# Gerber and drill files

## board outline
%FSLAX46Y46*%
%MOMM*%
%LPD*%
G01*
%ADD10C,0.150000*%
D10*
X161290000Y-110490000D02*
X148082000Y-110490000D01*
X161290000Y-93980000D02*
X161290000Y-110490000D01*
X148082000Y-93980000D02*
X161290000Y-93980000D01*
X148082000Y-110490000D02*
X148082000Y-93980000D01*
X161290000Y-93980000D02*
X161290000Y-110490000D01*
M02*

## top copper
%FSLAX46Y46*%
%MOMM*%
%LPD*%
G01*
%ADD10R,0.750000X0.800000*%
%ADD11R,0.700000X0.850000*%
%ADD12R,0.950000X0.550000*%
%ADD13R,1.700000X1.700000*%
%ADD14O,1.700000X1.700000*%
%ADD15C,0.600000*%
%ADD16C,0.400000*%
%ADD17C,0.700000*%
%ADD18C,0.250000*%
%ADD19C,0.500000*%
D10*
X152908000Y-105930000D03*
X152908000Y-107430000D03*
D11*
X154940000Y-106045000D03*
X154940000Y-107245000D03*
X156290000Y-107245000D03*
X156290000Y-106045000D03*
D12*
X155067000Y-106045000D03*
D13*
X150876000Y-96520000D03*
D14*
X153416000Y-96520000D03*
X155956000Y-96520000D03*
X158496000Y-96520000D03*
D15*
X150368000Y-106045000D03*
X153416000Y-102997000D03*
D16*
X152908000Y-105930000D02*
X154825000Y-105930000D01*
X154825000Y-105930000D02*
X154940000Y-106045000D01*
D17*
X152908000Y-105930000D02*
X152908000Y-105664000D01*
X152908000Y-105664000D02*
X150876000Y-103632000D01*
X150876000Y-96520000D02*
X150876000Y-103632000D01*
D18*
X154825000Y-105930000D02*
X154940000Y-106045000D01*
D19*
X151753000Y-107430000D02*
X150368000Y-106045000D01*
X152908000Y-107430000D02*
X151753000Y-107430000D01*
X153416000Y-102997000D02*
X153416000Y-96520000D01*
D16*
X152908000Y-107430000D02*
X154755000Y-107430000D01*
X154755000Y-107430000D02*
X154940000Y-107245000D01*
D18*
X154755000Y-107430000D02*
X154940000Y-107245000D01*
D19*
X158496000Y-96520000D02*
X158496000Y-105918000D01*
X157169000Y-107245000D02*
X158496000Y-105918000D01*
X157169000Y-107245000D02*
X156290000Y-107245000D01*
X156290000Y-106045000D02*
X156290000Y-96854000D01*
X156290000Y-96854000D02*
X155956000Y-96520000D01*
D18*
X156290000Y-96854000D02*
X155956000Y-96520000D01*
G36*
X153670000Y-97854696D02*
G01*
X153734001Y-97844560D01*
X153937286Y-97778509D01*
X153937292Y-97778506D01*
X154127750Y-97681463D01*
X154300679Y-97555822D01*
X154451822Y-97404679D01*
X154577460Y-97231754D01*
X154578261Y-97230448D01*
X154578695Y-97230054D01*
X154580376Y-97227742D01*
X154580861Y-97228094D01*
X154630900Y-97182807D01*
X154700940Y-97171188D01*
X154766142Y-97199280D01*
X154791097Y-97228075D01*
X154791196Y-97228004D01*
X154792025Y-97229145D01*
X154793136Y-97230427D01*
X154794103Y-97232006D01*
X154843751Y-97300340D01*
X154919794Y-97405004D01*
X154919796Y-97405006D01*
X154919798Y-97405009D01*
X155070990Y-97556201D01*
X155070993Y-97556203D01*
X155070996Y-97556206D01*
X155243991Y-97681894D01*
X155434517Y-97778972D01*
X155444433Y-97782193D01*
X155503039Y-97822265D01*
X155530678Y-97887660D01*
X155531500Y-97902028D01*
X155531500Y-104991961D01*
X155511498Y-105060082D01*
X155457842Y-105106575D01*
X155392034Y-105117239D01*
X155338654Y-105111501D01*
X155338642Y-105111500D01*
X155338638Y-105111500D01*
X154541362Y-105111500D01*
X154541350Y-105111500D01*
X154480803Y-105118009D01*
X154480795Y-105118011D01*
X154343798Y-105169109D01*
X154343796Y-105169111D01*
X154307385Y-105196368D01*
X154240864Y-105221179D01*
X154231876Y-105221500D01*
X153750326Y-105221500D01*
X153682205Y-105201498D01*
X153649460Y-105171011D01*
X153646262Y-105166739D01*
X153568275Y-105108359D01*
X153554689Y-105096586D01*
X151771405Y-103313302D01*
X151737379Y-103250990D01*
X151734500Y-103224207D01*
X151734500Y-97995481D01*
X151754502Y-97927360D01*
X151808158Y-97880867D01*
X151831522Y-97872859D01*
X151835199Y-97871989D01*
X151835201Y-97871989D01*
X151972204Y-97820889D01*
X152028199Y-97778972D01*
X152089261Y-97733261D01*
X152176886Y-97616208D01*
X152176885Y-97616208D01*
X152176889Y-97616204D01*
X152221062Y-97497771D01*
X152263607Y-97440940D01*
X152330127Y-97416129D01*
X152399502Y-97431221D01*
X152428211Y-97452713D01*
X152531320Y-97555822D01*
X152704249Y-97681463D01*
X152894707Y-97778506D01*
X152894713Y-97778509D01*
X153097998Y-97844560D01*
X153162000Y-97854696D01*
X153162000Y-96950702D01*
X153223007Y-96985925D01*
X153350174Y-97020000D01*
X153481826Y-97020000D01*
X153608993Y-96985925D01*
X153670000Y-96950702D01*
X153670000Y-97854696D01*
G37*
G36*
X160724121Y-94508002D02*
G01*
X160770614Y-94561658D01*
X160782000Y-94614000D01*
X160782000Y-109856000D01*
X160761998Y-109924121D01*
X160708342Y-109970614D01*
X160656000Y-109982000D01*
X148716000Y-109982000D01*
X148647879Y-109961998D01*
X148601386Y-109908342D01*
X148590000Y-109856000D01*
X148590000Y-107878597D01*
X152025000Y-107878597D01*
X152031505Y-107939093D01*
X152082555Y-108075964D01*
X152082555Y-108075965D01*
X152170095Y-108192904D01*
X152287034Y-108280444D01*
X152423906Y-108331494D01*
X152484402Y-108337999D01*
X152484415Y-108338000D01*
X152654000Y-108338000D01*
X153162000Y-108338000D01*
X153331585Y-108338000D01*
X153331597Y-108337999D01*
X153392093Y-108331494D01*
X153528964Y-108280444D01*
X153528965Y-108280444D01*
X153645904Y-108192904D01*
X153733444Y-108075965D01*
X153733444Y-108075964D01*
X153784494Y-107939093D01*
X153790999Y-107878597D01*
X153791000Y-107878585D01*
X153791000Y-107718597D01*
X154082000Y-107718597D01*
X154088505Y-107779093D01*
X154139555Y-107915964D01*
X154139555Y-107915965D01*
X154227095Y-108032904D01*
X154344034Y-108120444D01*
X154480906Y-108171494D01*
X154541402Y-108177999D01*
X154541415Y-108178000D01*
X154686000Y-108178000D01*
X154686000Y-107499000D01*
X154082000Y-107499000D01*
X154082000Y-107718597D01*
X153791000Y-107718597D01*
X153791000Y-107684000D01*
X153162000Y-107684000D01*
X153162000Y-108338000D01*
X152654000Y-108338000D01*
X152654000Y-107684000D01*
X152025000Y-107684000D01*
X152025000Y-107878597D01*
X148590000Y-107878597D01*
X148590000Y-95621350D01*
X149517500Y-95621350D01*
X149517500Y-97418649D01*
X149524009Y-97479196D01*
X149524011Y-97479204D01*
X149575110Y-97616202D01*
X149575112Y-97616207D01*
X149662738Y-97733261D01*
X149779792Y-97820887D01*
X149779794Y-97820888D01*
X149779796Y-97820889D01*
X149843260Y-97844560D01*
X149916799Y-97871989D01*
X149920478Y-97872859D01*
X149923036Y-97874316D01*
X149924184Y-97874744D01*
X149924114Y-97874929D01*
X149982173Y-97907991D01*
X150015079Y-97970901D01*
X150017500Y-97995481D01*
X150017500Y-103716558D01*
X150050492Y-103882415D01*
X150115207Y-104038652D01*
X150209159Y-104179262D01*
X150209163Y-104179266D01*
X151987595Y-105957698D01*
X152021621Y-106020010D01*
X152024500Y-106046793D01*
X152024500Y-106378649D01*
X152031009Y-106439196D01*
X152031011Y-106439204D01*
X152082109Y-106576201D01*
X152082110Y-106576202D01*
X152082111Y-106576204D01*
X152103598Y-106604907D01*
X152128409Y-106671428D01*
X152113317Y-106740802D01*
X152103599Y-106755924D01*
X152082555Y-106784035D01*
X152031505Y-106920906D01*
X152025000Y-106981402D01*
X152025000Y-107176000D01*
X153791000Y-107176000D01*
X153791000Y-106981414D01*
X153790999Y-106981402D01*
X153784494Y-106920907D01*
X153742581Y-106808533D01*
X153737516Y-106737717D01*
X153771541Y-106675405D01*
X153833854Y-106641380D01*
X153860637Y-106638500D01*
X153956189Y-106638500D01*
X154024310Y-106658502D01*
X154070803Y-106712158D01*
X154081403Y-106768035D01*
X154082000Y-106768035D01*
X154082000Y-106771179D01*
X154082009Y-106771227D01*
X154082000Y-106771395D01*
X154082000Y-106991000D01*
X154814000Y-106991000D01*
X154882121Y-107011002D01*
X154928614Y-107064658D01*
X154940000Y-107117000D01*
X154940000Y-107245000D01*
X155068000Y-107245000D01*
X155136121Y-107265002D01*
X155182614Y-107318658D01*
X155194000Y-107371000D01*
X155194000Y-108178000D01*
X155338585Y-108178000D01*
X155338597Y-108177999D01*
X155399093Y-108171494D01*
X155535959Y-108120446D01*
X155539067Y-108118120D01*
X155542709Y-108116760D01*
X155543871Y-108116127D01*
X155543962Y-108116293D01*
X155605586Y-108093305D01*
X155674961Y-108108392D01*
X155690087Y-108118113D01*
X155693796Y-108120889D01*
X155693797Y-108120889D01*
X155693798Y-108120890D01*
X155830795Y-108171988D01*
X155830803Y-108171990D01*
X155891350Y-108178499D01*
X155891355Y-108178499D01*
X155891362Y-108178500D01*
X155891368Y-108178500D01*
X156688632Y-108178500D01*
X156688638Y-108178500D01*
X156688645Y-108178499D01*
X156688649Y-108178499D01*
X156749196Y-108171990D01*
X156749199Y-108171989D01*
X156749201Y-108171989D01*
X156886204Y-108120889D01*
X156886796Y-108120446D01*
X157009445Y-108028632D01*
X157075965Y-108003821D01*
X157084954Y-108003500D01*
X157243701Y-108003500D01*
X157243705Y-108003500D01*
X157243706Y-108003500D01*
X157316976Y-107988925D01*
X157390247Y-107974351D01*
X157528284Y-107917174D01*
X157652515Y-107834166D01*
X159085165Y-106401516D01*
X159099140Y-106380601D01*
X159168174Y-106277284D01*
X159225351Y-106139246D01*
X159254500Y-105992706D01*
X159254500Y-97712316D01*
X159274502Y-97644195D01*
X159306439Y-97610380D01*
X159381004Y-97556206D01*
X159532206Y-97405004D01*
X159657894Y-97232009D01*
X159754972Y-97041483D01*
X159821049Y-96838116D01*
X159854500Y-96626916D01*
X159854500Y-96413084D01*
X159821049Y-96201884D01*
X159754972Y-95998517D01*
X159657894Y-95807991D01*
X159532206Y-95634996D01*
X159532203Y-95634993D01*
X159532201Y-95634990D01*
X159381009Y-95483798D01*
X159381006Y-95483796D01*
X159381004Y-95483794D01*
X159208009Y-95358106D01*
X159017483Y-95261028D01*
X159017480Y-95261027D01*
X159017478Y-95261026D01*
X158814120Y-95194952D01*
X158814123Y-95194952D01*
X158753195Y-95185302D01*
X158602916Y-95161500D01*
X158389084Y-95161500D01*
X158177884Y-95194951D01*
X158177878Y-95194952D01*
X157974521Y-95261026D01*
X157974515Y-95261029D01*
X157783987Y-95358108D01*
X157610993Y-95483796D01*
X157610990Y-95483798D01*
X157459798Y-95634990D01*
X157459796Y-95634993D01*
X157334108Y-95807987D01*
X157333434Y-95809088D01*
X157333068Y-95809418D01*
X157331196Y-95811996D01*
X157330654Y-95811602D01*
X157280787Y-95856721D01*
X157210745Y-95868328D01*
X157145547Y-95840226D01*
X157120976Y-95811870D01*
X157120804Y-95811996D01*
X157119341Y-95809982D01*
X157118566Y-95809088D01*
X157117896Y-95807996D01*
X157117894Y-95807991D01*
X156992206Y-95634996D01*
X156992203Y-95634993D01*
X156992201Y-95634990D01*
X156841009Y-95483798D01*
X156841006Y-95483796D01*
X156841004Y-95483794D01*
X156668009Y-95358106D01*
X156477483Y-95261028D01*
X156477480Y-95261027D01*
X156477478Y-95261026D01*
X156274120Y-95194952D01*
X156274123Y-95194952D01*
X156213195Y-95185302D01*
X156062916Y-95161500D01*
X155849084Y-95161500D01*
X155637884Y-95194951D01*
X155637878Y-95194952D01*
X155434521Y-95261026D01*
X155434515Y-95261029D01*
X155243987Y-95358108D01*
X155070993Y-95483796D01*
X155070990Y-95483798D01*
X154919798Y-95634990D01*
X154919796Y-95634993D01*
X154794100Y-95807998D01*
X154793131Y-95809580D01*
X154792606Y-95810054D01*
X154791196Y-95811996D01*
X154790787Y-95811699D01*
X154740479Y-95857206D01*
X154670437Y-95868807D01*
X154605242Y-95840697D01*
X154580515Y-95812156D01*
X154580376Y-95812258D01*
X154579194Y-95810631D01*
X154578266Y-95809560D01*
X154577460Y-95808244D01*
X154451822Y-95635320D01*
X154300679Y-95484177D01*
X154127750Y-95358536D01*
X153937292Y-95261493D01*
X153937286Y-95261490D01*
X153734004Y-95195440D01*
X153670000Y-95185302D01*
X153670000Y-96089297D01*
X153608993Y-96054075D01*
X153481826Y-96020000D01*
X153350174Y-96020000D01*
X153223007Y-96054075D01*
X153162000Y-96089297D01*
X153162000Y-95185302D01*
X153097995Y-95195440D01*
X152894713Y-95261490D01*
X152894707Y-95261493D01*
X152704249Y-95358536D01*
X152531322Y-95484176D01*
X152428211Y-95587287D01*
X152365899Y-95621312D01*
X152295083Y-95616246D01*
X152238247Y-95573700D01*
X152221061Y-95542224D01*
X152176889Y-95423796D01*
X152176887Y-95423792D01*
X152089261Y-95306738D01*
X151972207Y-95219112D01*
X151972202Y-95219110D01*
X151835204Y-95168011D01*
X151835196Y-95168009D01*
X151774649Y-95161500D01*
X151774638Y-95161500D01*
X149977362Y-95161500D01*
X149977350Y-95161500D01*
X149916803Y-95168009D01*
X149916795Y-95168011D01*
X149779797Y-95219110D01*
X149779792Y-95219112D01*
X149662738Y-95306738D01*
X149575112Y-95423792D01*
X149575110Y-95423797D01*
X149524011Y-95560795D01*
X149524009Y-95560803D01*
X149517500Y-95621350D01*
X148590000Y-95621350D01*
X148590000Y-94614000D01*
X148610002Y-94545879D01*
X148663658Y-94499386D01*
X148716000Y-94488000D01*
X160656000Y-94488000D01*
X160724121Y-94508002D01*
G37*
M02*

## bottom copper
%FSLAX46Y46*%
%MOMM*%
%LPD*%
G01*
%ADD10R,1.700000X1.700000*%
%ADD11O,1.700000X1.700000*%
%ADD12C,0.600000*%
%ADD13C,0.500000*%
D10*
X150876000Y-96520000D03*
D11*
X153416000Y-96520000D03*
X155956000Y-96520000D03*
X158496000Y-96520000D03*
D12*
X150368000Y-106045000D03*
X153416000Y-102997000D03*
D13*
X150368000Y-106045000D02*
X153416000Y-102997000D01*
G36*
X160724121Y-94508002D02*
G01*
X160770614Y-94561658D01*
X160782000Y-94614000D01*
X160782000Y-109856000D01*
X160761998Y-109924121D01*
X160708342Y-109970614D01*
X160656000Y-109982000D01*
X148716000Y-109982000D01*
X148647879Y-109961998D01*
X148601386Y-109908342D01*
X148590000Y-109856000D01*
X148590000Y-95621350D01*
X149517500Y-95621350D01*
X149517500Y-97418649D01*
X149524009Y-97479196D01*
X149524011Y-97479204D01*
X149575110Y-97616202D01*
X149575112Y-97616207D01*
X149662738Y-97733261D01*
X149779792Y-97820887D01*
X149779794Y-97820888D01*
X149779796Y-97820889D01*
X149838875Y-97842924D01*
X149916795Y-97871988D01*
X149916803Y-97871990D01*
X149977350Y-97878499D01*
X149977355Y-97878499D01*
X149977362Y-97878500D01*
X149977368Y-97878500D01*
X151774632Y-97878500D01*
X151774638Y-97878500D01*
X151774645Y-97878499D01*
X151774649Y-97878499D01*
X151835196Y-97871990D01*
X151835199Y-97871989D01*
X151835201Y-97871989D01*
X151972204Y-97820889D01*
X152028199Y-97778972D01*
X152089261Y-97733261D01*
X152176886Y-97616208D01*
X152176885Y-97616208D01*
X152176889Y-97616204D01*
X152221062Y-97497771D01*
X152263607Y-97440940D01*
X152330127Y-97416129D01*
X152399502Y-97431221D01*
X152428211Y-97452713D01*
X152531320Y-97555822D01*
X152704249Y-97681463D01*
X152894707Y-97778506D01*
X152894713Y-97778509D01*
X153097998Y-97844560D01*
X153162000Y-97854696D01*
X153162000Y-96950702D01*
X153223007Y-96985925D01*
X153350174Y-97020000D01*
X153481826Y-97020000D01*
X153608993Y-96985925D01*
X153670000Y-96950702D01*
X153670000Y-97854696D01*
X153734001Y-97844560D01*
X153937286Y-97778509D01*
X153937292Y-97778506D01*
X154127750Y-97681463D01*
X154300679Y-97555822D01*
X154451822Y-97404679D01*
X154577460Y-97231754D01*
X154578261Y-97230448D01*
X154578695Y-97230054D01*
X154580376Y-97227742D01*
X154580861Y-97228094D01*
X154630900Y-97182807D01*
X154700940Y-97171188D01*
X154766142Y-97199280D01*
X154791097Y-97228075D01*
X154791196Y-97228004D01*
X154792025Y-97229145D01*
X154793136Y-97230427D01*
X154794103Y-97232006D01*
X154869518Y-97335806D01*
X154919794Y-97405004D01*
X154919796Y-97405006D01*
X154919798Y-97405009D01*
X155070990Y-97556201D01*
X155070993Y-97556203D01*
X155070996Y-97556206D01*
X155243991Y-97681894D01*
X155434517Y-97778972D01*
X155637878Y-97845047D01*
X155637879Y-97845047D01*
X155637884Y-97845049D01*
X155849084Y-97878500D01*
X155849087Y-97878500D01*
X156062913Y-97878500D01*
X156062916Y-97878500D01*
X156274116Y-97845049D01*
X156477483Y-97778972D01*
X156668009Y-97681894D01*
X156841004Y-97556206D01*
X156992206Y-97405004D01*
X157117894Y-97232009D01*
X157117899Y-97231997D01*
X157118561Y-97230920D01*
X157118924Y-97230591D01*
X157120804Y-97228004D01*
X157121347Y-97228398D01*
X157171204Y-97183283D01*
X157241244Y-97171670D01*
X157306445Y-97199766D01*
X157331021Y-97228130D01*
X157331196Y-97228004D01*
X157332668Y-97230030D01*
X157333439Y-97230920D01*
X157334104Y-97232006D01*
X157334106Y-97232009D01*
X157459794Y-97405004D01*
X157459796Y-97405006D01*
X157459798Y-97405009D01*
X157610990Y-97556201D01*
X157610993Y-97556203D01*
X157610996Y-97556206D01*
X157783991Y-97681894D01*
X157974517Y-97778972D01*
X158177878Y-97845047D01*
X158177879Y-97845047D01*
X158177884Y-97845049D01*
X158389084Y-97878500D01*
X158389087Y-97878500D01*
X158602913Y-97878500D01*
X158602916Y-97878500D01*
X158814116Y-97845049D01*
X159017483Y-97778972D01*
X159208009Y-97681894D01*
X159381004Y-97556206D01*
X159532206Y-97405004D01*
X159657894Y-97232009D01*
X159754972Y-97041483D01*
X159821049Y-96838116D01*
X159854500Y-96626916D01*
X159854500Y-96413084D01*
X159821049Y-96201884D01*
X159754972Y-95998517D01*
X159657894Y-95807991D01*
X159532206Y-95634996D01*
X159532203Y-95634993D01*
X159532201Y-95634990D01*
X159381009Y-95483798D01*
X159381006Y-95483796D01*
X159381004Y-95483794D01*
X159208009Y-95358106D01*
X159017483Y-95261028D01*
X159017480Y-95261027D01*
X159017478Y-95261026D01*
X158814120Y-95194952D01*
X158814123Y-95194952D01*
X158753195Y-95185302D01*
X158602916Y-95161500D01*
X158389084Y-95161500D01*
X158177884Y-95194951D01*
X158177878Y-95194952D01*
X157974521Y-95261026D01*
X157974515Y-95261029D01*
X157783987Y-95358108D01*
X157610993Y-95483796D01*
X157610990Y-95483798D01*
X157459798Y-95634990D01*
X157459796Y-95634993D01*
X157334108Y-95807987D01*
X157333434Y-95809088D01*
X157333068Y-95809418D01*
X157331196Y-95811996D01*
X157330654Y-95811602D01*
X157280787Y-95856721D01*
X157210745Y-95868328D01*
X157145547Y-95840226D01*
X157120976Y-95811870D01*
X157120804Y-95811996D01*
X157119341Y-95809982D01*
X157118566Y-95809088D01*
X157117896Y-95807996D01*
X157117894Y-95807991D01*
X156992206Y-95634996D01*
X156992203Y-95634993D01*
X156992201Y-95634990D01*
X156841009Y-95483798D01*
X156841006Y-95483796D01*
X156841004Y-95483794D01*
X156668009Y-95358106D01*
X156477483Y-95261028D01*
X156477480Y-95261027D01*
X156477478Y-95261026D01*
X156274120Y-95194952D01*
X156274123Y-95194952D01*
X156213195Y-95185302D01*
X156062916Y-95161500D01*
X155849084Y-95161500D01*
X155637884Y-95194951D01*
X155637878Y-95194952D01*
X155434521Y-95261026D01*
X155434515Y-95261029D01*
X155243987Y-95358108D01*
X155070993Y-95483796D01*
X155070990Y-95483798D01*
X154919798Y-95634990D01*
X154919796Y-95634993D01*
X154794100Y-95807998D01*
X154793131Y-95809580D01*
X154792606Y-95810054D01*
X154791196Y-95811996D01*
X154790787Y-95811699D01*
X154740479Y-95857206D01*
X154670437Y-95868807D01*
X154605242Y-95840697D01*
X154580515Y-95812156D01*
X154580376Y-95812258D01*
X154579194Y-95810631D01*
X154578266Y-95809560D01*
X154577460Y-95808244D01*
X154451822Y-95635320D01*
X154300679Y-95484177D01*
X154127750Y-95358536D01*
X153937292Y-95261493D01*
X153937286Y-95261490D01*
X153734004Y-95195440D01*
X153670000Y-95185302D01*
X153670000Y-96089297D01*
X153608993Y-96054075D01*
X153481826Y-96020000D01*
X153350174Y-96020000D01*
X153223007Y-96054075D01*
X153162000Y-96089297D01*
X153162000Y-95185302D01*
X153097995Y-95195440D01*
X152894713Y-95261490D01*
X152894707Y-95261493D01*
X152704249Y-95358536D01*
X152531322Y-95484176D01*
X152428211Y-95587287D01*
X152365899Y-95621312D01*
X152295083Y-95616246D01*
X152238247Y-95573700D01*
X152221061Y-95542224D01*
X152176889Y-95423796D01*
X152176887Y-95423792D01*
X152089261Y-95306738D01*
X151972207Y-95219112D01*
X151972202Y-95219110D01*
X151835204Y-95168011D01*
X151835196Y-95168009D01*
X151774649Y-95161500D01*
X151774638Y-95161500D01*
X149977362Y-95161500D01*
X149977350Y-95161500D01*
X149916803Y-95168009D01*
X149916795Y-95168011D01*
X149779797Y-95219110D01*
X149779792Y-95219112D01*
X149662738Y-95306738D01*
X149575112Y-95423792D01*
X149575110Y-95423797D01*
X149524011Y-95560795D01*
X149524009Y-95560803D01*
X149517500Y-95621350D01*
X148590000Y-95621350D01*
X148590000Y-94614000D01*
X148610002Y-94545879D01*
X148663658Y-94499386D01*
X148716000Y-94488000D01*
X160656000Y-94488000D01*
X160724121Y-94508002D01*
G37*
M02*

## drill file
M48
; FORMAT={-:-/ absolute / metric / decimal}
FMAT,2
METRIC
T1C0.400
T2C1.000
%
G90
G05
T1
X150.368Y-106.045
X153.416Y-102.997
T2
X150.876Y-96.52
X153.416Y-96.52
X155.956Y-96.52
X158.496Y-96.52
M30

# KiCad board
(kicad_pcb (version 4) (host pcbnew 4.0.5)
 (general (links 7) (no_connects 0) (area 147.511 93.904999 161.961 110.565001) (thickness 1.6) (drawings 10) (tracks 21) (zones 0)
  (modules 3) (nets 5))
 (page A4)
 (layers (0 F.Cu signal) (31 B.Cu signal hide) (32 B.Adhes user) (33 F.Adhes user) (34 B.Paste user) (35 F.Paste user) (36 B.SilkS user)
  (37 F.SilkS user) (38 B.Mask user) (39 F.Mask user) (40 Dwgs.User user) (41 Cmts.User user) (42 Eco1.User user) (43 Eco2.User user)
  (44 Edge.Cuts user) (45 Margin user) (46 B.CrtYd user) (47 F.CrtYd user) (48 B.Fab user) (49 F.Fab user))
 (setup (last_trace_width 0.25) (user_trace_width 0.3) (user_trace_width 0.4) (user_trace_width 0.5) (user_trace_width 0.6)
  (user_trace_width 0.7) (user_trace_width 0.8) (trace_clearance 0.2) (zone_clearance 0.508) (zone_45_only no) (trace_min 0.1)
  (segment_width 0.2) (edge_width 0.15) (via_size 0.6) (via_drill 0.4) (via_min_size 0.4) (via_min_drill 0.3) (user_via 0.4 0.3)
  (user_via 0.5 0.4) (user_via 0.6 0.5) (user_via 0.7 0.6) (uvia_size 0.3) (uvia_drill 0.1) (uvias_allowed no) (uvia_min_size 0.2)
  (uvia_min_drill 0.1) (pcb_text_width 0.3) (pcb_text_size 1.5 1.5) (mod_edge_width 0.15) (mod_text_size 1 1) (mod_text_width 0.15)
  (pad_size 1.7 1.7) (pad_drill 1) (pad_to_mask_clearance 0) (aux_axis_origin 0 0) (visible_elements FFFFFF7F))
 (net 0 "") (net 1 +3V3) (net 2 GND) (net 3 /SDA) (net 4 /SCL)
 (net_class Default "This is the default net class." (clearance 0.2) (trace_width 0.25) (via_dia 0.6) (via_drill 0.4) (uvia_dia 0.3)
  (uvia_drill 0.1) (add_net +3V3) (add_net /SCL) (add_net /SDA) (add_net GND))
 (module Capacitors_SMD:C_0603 (layer F.Cu) (at 152.908 106.68 270)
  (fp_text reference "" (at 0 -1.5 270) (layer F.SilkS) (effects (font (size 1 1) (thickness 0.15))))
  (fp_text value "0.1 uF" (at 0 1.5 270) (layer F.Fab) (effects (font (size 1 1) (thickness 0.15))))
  (pad 1 smd rect (at -0.75 0 270) (size 0.8 0.75) (layers F.Cu F.Paste F.Mask) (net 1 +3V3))
  (pad 2 smd rect (at 0.75 0 270) (size 0.8 0.75) (layers F.Cu F.Paste F.Mask) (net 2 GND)))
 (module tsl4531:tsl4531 (layer F.Cu) (at 154.94 106.045)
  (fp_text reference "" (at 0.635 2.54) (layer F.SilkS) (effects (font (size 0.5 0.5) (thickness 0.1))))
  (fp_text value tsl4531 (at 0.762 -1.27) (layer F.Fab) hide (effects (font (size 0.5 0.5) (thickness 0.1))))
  (pad 1 smd rect (at 0 0) (size 0.7 0.85) (layers F.Cu F.Paste F.Mask) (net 1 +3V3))
  (pad 2 smd rect (at 0 1.2) (size 0.7 0.85) (layers F.Cu F.Paste F.Mask) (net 2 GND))
  (pad 3 smd rect (at 1.35 1.2) (size 0.7 0.85) (layers F.Cu F.Paste F.Mask) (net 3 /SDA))
  (pad 4 smd rect (at 1.35 0) (size 0.7 0.85) (layers F.Cu F.Paste F.Mask) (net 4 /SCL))
  (pad 1 smd rect (at 0.127 0) (size 0.95 0.55) (layers F.Cu F.Paste F.Mask) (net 1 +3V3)))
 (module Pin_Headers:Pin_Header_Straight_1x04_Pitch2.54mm (layer F.Cu) (at 150.876 96.52 90)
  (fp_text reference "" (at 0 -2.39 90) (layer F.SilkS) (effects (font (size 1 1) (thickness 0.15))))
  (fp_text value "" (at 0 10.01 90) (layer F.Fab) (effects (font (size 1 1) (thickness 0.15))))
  (pad 1 thru_hole rect (at 0 0 90) (size 1.7 1.7) (drill 1) (layers *.Cu *.Mask) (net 1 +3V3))
  (pad 2 thru_hole oval (at 0 2.54 90) (size 1.7 1.7) (drill 1) (layers *.Cu *.Mask) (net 2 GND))
  (pad 3 thru_hole oval (at 0 5.08 90) (size 1.7 1.7) (drill 1) (layers *.Cu *.Mask) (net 4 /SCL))
  (pad 4 thru_hole oval (at 0 7.62 90) (size 1.7 1.7) (drill 1) (layers *.Cu *.Mask) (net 3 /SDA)))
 (gr_line (start 161.29 110.49) (end 148.082 110.49) (angle 90) (layer Edge.Cuts) (width 0.15))
 (gr_line (start 161.29 93.98) (end 161.29 110.49) (angle 90) (layer Edge.Cuts) (width 0.15))
 (gr_line (start 148.082 93.98) (end 161.29 93.98) (angle 90) (layer Edge.Cuts) (width 0.15))
 (gr_line (start 148.082 110.49) (end 148.082 93.98) (angle 90) (layer Edge.Cuts) (width 0.15))
 (gr_line (start 161.29 93.98) (end 161.29 110.49) (angle 90) (layer Edge.Cuts) (width 0.15))
 (segment (start 152.908 105.93) (end 154.825 105.93) (width 0.4) (layer F.Cu) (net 1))
 (segment (start 154.825 105.93) (end 154.94 106.045) (width 0.4) (layer F.Cu) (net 1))
 (segment (start 152.908 105.93) (end 152.908 105.664) (width 0.7) (layer F.Cu) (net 1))
 (segment (start 152.908 105.664) (end 150.876 103.632) (width 0.7) (layer F.Cu) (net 1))
 (segment (start 150.876 96.52) (end 150.876 103.632) (width 0.7) (layer F.Cu) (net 1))
 (segment (start 154.825 105.93) (end 154.94 106.045) (width 0.25) (layer F.Cu) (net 1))
 (segment (start 150.368 106.045) (end 153.416 102.997) (width 0.5) (layer B.Cu) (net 2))
 (segment (start 151.753 107.43) (end 150.368 106.045) (width 0.5) (layer F.Cu) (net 2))
 (via (at 150.368 106.045) (size 0.6) (drill 0.4) (layers F.Cu B.Cu) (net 2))
 (segment (start 152.908 107.43) (end 151.753 107.43) (width 0.5) (layer F.Cu) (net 2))
 (segment (start 153.416 102.997) (end 153.416 96.52) (width 0.5) (layer F.Cu) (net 2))
 (via (at 153.416 102.997) (size 0.6) (drill 0.4) (layers F.Cu B.Cu) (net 2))
 (segment (start 152.908 107.43) (end 154.755 107.43) (width 0.4) (layer F.Cu) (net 2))
 (segment (start 154.755 107.43) (end 154.94 107.245) (width 0.4) (layer F.Cu) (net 2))
 (segment (start 154.755 107.43) (end 154.94 107.245) (width 0.25) (layer F.Cu) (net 2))
 (segment (start 158.496 96.52) (end 158.496 105.918) (width 0.5) (layer F.Cu) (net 3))
 (segment (start 157.169 107.245) (end 158.496 105.918) (width 0.5) (layer F.Cu) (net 3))
 (segment (start 157.169 107.245) (end 156.29 107.245) (width 0.5) (layer F.Cu) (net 3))
 (segment (start 156.29 106.045) (end 156.29 96.854) (width 0.5) (layer F.Cu) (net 4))
 (segment (start 156.29 96.854) (end 155.956 96.52) (width 0.5) (layer F.Cu) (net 4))
 (segment (start 156.29 96.854) (end 155.956 96.52) (width 0.25) (layer F.Cu) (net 4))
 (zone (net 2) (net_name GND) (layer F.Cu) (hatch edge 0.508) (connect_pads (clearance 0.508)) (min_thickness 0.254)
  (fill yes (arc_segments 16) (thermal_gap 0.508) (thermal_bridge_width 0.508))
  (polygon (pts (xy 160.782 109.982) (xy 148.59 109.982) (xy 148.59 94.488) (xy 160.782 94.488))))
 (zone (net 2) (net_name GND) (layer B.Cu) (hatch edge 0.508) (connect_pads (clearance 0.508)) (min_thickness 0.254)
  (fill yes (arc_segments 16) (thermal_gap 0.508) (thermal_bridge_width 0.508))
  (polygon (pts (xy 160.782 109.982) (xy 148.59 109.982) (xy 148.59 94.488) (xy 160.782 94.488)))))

